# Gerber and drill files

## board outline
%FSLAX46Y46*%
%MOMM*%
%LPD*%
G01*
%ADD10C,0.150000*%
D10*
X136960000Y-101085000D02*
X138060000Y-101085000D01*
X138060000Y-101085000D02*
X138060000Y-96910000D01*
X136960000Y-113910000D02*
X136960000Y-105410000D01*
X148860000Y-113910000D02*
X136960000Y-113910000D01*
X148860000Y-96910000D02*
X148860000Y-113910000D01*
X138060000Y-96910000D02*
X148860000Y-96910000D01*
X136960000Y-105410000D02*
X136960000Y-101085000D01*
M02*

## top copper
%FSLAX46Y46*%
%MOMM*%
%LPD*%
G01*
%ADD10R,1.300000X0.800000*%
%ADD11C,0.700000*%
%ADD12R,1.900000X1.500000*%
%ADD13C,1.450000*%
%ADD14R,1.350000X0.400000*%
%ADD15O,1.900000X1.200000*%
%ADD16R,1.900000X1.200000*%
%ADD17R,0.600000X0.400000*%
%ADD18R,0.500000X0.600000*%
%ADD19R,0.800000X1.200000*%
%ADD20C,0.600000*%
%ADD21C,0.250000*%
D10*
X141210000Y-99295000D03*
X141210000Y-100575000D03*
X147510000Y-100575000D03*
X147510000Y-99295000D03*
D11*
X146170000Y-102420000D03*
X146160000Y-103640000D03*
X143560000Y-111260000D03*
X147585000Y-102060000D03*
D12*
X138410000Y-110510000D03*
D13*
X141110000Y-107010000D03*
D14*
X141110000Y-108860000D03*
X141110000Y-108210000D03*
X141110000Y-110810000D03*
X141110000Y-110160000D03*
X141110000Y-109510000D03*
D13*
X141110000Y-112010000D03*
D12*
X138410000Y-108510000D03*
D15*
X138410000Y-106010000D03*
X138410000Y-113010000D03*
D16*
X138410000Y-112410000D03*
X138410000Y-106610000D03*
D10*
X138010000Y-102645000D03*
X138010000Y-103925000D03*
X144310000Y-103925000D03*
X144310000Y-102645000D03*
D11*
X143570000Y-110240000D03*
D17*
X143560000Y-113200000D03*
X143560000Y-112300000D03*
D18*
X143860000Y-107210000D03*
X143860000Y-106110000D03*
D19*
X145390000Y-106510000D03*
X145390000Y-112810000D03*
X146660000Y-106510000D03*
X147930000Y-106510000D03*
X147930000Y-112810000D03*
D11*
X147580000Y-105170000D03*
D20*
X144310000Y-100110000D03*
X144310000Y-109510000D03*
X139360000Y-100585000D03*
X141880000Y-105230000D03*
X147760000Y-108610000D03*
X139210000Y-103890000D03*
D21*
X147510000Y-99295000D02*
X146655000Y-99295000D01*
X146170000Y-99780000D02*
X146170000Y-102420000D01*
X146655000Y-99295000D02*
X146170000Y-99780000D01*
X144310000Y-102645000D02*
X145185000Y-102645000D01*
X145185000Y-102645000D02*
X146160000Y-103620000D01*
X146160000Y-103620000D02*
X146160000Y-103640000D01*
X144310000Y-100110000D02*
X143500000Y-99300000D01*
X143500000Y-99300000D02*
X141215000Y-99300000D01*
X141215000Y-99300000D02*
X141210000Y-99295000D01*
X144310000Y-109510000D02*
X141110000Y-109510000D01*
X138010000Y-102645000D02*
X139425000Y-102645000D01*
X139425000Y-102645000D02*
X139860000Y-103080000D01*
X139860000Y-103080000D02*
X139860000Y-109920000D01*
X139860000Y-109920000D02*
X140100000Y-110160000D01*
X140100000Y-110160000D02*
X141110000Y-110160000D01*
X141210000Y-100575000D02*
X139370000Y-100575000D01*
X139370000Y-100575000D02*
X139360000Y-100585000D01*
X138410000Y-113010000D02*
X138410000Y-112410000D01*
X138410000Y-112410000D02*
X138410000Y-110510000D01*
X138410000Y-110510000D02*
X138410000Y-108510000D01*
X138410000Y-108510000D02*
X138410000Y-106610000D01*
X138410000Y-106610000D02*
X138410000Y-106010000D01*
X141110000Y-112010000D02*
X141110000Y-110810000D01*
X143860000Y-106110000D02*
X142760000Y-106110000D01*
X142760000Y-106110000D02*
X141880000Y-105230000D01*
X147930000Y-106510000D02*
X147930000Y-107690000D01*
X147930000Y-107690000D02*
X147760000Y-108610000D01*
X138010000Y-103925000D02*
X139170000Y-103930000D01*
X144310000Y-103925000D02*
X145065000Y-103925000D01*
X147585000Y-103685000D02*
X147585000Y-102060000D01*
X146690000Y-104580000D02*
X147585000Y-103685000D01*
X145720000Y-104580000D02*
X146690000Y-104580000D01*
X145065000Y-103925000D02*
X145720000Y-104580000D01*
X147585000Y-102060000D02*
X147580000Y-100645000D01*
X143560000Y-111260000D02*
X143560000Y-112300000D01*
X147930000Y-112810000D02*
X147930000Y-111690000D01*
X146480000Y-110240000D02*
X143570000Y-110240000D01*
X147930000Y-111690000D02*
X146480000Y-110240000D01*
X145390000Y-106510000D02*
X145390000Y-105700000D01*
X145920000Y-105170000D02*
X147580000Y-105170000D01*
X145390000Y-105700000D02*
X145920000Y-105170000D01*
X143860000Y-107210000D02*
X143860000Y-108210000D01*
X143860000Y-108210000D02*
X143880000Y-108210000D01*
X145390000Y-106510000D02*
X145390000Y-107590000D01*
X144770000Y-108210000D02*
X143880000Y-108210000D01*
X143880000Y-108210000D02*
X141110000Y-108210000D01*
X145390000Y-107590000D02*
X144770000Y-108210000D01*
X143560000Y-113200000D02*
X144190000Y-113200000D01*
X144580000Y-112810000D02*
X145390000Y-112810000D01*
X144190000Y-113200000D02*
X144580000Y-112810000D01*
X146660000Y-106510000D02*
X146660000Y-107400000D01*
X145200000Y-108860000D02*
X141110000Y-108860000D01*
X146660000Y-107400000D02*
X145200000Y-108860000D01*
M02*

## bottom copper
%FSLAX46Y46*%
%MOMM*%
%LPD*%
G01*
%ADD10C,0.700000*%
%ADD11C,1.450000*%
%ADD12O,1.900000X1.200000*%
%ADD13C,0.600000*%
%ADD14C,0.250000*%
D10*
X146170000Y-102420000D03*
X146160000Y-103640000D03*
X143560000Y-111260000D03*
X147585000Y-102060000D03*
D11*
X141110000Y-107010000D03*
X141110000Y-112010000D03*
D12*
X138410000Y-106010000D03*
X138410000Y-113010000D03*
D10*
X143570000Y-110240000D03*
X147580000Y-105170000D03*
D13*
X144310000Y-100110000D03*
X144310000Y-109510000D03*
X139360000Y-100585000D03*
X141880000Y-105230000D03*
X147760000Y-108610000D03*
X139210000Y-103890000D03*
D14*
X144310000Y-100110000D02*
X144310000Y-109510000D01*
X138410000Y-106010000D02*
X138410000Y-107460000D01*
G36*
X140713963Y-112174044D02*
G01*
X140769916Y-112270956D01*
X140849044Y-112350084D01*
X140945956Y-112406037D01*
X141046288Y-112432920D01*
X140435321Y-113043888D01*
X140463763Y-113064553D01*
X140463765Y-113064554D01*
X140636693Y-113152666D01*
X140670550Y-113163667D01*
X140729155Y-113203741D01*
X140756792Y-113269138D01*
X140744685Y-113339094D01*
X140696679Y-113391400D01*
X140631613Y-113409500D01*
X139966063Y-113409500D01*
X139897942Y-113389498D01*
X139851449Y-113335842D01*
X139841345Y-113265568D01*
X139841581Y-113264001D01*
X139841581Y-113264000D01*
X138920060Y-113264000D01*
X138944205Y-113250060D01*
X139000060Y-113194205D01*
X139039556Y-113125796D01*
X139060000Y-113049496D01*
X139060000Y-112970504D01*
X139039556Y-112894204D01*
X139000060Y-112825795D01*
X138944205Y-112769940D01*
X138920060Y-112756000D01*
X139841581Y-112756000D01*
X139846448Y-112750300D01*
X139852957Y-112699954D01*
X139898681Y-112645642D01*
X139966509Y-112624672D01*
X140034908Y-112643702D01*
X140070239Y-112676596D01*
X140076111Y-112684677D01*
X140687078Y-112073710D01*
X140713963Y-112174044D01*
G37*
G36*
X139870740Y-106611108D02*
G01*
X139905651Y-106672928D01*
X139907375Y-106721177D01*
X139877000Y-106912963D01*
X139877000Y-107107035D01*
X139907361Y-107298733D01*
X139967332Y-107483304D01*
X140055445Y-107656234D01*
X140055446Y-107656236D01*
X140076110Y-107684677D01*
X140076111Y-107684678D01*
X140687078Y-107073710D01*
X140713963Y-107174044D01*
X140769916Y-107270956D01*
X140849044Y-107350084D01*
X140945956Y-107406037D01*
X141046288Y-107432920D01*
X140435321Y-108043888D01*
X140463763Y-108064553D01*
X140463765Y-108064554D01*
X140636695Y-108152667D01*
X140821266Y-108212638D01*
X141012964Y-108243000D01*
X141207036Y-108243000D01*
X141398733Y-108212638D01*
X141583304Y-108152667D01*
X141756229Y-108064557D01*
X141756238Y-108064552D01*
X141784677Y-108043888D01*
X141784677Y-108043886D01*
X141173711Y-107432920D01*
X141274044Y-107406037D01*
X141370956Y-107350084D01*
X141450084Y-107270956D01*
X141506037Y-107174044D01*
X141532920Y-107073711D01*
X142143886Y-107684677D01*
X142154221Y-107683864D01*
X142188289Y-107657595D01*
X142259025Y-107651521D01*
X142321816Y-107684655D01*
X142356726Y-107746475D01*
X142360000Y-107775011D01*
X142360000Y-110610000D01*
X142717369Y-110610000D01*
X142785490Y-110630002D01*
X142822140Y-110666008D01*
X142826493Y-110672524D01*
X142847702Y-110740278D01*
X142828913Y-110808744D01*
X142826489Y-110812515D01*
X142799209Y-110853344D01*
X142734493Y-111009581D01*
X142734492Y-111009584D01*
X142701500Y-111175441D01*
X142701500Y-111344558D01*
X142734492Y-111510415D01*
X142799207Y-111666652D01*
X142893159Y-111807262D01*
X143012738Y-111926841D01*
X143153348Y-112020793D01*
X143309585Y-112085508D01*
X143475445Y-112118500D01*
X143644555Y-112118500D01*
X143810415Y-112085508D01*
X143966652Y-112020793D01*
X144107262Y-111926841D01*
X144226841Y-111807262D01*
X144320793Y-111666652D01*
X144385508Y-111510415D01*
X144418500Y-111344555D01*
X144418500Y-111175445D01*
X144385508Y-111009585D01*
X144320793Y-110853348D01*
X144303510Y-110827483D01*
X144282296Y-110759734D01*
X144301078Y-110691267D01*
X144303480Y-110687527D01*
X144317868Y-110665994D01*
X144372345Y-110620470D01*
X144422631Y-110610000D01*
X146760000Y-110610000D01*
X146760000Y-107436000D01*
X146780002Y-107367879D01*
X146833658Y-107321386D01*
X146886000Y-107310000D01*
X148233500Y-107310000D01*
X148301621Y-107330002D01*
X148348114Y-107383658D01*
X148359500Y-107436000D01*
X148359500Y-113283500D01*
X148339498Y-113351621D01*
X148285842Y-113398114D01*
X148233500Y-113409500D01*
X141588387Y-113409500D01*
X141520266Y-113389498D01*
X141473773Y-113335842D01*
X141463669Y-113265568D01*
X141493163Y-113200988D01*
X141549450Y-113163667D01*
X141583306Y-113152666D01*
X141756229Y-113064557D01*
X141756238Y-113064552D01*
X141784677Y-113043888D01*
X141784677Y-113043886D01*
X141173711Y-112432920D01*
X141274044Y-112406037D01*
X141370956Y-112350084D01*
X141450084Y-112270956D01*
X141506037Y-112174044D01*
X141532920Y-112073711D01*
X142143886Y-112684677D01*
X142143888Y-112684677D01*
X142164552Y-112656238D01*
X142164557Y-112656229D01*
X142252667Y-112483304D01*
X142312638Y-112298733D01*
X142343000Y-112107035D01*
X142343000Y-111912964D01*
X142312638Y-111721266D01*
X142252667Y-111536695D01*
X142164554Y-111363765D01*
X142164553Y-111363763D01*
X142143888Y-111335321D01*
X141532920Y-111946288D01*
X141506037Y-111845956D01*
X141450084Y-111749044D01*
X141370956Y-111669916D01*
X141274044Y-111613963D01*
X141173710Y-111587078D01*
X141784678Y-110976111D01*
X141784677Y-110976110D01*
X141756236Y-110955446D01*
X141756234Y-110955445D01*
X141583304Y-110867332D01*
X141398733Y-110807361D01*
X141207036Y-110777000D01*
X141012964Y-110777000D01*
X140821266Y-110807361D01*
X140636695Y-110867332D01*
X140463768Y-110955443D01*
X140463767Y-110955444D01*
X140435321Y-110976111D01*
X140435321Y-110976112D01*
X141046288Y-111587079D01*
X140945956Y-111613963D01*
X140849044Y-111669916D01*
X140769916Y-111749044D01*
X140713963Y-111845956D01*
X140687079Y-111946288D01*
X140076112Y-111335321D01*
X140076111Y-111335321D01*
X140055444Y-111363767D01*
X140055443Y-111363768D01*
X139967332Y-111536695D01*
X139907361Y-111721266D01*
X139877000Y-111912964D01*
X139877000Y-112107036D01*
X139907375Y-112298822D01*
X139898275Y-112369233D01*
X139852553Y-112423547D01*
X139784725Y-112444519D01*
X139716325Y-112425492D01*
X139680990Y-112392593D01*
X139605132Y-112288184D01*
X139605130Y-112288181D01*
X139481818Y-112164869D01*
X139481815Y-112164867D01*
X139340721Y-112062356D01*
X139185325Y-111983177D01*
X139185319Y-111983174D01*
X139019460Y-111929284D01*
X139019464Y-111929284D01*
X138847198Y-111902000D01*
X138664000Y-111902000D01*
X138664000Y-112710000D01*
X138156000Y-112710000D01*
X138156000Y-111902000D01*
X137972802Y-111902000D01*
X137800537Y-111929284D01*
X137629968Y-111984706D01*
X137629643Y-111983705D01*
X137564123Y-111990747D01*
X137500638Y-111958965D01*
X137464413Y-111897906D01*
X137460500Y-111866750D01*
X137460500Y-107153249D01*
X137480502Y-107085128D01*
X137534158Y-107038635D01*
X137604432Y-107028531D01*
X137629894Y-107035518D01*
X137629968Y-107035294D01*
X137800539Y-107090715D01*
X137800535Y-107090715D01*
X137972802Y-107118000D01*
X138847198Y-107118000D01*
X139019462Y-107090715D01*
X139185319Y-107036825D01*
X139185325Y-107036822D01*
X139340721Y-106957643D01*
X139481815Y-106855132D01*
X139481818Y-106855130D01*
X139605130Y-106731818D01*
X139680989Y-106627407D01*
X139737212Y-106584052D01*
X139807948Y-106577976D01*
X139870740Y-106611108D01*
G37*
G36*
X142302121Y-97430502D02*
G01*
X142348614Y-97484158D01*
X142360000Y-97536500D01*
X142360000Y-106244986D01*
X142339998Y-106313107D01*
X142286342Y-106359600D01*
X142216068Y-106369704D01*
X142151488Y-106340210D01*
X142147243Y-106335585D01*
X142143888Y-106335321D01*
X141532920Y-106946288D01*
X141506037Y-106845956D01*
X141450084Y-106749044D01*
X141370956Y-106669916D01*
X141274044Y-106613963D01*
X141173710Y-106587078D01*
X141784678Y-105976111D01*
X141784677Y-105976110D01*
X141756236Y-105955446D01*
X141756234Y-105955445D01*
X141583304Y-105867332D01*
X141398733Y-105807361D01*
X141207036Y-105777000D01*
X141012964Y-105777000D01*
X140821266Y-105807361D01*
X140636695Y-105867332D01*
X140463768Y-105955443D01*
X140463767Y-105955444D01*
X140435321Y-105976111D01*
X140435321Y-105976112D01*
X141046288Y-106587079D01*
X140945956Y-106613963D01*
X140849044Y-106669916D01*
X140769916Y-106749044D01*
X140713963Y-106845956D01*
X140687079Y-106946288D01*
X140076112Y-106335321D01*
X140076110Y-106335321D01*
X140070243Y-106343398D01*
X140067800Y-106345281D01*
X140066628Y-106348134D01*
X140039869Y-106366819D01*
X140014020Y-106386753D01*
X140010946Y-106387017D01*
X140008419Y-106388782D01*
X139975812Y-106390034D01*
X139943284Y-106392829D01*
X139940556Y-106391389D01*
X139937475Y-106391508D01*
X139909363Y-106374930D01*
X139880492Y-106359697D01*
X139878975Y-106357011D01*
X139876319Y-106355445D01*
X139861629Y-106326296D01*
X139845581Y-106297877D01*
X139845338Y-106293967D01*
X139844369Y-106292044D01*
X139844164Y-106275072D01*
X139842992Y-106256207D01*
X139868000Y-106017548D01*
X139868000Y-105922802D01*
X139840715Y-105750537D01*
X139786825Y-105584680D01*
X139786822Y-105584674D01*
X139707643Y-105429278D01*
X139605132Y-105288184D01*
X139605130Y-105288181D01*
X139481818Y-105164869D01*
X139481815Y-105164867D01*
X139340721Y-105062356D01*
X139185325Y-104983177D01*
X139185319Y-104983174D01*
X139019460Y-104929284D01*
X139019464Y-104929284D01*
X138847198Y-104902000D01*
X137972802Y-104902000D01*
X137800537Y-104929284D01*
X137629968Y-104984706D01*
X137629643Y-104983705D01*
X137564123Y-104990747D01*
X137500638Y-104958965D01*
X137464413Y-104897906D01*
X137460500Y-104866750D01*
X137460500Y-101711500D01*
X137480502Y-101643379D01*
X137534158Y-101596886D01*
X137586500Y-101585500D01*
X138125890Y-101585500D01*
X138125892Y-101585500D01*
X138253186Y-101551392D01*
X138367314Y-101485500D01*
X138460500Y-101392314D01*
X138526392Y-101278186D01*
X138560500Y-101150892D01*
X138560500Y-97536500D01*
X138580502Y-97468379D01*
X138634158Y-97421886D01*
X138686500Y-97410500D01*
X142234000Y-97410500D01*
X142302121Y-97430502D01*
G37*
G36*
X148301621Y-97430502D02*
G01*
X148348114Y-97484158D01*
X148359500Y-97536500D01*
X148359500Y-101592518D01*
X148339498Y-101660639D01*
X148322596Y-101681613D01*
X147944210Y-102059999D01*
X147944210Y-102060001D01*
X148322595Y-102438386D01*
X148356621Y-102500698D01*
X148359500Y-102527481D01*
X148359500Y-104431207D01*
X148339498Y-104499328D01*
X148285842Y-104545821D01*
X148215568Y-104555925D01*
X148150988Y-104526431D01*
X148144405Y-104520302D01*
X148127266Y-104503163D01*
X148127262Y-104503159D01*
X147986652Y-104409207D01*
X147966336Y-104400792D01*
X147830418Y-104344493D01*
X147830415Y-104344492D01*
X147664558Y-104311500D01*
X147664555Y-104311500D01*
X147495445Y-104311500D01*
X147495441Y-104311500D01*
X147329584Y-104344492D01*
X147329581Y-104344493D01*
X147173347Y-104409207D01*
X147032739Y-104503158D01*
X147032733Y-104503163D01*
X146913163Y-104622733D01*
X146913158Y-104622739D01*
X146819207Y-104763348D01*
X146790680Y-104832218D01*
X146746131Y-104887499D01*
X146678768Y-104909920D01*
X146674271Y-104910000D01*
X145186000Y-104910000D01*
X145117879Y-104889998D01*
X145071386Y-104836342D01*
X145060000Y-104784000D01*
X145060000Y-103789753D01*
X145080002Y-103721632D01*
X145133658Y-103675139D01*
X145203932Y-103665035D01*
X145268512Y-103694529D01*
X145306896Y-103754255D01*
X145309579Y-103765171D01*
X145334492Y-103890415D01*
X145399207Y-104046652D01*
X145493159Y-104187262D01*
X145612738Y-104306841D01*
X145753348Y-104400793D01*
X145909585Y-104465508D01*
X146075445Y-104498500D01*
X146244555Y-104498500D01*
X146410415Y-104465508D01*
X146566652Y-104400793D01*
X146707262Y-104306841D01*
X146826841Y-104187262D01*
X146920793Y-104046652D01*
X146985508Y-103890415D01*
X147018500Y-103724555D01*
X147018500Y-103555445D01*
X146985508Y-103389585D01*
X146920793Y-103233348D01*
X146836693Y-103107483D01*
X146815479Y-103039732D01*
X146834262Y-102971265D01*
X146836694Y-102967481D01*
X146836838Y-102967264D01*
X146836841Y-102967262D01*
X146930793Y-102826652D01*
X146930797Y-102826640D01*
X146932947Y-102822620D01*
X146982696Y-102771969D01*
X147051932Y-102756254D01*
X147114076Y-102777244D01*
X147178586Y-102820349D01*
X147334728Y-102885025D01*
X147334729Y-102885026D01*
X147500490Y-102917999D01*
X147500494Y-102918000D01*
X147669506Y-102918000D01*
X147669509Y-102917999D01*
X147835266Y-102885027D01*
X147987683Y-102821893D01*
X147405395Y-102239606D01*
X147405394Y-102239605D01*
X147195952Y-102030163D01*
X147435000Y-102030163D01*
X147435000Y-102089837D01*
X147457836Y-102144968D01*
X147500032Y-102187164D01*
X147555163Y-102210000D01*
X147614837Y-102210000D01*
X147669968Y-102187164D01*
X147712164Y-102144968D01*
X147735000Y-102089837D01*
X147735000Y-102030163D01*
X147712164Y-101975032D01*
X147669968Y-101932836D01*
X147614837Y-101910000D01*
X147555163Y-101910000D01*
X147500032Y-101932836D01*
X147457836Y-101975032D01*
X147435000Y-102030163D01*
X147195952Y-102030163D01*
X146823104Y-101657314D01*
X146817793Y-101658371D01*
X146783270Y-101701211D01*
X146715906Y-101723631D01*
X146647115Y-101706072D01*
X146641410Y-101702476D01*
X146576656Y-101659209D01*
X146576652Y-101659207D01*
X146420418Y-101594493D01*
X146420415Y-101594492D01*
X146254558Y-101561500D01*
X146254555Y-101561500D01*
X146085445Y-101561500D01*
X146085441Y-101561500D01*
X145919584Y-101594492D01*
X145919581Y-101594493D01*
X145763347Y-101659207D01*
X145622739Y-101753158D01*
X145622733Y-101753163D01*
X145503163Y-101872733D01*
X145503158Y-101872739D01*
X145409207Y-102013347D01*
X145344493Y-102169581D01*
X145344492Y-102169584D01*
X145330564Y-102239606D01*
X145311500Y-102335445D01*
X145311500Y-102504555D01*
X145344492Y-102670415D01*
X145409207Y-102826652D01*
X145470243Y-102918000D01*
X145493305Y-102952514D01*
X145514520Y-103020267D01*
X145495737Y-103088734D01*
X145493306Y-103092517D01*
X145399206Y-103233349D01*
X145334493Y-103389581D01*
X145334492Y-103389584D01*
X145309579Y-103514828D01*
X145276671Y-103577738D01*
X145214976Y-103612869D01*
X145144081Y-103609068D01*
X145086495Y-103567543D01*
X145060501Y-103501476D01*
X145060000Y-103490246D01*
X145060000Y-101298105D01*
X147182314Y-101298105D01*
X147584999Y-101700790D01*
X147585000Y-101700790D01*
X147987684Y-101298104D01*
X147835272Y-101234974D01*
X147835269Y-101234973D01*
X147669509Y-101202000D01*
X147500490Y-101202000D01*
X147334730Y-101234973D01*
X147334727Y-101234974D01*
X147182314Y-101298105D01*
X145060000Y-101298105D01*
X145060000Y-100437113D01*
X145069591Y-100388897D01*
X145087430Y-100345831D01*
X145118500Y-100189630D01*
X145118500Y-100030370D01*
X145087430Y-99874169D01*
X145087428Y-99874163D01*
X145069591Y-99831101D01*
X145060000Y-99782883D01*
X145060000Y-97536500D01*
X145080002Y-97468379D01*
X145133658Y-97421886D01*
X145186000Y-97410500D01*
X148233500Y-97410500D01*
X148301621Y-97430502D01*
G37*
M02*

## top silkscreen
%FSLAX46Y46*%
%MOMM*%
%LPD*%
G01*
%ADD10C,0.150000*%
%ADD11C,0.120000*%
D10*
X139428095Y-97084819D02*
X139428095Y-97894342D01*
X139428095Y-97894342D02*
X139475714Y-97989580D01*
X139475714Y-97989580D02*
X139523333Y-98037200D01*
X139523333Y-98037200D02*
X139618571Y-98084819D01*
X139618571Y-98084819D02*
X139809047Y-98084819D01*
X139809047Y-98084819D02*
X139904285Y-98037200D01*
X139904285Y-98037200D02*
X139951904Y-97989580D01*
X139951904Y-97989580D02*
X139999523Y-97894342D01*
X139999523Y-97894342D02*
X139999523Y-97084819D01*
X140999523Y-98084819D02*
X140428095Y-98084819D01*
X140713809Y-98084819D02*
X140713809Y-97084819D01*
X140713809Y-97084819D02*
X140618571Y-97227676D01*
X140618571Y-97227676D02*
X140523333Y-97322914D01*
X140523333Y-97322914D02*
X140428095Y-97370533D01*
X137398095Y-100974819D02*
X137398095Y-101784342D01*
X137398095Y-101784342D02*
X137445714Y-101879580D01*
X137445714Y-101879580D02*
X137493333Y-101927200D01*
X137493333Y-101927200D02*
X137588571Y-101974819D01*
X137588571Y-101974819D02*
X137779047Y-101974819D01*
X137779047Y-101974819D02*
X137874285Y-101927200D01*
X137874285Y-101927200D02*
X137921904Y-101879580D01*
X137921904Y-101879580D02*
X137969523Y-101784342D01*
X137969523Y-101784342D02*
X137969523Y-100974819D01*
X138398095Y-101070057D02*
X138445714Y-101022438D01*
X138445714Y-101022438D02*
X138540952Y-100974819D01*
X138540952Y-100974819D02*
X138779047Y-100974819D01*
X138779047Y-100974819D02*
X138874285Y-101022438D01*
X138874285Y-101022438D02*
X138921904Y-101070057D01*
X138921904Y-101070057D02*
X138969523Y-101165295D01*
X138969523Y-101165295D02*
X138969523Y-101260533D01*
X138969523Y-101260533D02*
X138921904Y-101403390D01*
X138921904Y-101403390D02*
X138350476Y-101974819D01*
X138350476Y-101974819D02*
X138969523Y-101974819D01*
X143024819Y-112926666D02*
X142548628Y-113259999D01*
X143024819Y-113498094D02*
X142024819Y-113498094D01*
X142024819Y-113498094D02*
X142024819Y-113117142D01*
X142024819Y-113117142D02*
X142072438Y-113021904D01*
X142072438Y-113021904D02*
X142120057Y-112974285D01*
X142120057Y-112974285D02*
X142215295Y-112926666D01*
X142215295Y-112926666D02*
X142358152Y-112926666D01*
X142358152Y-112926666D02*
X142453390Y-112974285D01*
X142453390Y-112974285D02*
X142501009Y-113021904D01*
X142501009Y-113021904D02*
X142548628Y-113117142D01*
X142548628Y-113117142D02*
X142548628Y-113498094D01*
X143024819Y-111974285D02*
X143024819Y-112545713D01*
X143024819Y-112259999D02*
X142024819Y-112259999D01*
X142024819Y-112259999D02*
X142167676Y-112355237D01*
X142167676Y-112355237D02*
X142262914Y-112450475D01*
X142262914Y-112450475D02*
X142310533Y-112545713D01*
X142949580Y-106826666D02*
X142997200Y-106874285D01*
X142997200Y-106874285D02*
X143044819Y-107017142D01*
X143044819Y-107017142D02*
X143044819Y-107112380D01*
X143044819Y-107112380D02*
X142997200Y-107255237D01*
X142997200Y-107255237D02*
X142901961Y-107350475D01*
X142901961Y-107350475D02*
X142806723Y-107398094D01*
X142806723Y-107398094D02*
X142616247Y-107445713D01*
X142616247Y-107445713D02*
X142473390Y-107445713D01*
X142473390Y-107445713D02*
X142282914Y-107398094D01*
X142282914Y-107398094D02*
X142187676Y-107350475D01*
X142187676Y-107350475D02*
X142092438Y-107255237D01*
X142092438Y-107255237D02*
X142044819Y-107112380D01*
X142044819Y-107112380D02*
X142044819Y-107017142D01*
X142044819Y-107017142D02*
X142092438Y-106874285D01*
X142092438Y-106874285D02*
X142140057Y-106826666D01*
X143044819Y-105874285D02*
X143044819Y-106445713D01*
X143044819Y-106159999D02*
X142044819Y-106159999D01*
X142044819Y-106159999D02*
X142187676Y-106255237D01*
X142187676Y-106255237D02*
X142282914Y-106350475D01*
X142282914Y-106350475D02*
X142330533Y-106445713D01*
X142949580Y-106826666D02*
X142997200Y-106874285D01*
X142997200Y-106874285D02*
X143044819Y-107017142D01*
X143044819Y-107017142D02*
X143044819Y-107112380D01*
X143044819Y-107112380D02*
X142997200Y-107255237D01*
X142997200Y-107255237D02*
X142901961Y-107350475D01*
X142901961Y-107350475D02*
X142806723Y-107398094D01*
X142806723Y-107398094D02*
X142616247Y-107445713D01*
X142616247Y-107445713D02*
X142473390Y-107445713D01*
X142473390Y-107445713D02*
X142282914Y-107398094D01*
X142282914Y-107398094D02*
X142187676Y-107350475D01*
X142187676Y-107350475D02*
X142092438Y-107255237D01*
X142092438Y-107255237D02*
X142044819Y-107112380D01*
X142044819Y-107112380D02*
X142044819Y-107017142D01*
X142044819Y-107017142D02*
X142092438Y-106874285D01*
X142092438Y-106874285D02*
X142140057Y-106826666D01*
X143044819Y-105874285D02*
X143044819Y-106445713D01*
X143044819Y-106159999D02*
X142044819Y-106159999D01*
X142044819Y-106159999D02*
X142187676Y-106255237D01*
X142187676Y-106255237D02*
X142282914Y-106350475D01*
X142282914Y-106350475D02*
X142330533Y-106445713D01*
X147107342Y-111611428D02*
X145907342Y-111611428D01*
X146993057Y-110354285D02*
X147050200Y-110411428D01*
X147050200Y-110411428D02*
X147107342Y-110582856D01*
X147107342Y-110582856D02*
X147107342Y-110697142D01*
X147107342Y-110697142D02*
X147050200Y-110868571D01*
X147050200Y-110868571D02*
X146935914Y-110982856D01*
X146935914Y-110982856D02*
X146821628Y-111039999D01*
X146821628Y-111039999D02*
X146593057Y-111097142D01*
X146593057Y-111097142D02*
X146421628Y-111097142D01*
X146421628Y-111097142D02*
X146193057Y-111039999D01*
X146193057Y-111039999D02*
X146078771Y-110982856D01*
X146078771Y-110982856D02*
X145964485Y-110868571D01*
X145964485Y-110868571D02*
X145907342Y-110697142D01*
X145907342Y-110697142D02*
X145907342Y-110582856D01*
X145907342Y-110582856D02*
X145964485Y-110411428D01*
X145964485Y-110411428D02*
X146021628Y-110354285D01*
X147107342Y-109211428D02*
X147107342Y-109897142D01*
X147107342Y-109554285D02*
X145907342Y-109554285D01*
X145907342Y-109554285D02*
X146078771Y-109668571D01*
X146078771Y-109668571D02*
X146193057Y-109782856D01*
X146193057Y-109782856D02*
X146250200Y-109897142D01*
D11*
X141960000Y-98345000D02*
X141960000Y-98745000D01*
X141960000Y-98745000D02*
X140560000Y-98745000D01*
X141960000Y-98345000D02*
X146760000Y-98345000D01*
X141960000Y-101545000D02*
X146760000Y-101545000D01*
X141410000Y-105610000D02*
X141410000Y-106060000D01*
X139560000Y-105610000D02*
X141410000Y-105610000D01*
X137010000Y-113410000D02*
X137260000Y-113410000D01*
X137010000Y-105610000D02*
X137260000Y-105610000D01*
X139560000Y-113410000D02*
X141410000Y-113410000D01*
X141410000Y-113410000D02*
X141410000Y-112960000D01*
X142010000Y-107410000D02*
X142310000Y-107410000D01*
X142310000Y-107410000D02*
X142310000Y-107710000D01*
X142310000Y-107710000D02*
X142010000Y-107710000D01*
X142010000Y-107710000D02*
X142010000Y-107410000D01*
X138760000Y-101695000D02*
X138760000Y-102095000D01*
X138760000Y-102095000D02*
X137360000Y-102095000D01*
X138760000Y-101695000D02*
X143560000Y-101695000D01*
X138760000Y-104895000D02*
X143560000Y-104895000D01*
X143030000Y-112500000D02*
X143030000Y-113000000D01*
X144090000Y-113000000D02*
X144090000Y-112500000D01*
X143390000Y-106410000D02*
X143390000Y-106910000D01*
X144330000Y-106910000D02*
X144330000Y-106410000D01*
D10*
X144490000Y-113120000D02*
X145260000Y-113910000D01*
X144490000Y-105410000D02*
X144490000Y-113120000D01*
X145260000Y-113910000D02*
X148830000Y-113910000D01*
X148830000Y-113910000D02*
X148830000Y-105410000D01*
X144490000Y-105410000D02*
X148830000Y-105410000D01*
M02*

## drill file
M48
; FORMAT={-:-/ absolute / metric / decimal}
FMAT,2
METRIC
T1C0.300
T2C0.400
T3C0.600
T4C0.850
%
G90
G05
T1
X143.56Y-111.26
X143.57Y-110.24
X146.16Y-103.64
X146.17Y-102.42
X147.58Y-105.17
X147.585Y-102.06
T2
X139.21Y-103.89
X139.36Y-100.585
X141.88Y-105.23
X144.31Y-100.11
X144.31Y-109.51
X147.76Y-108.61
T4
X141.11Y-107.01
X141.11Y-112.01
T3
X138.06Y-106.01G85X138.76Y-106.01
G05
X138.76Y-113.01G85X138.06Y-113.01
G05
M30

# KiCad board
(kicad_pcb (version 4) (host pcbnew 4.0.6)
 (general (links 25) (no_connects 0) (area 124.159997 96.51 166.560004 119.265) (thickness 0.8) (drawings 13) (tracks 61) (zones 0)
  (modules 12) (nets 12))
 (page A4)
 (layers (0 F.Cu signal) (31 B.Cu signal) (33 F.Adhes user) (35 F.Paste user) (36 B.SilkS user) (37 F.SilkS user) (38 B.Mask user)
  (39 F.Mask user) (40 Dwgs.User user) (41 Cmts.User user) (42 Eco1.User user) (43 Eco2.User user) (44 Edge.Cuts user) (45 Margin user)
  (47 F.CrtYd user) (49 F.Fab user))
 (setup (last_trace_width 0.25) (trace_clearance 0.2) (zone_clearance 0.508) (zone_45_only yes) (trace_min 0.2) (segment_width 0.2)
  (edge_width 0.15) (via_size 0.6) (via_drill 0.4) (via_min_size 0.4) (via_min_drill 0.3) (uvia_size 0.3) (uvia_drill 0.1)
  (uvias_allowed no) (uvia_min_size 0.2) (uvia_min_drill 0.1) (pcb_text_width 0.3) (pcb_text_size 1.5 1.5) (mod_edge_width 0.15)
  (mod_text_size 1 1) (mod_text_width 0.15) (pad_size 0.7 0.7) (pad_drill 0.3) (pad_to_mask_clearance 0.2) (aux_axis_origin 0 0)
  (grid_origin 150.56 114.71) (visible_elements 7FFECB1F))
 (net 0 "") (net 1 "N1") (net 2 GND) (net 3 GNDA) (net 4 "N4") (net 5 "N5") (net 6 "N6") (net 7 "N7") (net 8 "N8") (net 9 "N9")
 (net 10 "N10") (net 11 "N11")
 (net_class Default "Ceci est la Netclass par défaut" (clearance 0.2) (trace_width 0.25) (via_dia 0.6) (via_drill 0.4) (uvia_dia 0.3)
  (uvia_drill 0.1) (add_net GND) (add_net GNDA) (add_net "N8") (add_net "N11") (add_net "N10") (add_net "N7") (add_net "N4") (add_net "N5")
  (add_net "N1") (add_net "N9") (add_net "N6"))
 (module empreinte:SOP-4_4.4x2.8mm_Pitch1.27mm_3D (layer F.Cu) (at 144.36 99.935)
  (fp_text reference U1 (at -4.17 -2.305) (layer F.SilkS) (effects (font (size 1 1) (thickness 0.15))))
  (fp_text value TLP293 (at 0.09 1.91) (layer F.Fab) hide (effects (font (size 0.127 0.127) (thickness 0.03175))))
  (fp_line (start -2.4 -1.59) (end -2.4 -1.19) (layer F.SilkS) (width 0.12))
  (fp_line (start -2.4 -1.19) (end -3.8 -1.19) (layer F.SilkS) (width 0.12))
  (fp_line (start -2.4 -1.59) (end 2.4 -1.59) (layer F.SilkS) (width 0.12))
  (fp_line (start -2.4 1.61) (end 2.4 1.61) (layer F.SilkS) (width 0.12))
  (pad 1 smd rect (at -3.15 -0.64) (size 1.3 0.8) (layers F.Cu F.Paste F.Mask) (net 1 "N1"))
  (pad 2 smd rect (at -3.15 0.64) (size 1.3 0.8) (layers F.Cu F.Paste F.Mask) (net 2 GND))
  (pad 3 smd rect (at 3.15 0.64) (size 1.3 0.8) (layers F.Cu F.Paste F.Mask) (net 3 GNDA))
  (pad 4 smd rect (at 3.15 -0.64) (size 1.3 0.8) (layers F.Cu F.Paste F.Mask) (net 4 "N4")))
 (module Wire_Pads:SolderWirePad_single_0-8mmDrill (layer F.Cu) (at 146.17 102.42)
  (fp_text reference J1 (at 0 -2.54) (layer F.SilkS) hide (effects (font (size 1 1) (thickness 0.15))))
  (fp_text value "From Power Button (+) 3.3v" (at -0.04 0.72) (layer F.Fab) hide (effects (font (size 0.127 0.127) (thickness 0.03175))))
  (pad 1 thru_hole circle (at 0 0) (size 0.7 0.7) (drill 0.3) (layers *.Cu *.Mask) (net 4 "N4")))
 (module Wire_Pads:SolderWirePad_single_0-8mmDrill (layer F.Cu) (at 146.16 103.64)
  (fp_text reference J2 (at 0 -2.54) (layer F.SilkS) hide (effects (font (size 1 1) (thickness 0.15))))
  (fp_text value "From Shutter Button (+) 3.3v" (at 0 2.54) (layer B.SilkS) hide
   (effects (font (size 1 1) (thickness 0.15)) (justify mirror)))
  (pad 1 thru_hole circle (at 0 0) (size 0.7 0.7) (drill 0.3) (layers *.Cu *.Mask) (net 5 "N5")))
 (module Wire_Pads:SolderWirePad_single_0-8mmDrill (layer F.Cu) (at 143.56 111.26)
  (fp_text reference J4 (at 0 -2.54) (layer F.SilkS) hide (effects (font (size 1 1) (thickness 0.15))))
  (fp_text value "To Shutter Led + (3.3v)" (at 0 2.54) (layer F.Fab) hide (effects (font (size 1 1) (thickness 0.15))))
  (pad 1 thru_hole circle (at 0 0) (size 0.7 0.7) (drill 0.3) (layers *.Cu *.Mask) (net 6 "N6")))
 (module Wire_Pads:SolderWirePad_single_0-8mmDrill (layer F.Cu) (at 147.585 102.06)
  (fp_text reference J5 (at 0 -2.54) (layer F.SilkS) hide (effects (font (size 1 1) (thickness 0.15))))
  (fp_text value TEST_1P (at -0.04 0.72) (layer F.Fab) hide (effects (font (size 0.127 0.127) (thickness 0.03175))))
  (pad 1 thru_hole circle (at 0 0) (size 0.7 0.7) (drill 0.3) (layers *.Cu *.Mask) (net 3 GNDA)))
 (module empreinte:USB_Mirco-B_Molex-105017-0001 (layer F.Cu) (at 141.11 109.51 270)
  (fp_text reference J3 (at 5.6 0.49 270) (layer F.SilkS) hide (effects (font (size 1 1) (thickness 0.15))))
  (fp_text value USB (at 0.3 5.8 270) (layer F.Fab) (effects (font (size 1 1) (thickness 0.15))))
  (fp_line (start -3.9 -0.3) (end -3.45 -0.3) (layer F.SilkS) (width 0.12))
  (fp_line (start -3.9 1.55) (end -3.9 -0.3) (layer F.SilkS) (width 0.12))
  (fp_line (start 3.9 4.1) (end 3.9 3.85) (layer F.SilkS) (width 0.12))
  (fp_line (start -3.9 4.1) (end -3.9 3.85) (layer F.SilkS) (width 0.12))
  (fp_line (start 3.9 1.55) (end 3.9 -0.3) (layer F.SilkS) (width 0.12))
  (fp_line (start 3.9 -0.3) (end 3.45 -0.3) (layer F.SilkS) (width 0.12))
  (fp_line (start -2.1 -0.9) (end -2.1 -1.2) (layer F.SilkS) (width 0.12))
  (fp_line (start -2.1 -1.2) (end -1.8 -1.2) (layer F.SilkS) (width 0.12))
  (fp_line (start -1.8 -1.2) (end -1.8 -0.9) (layer F.SilkS) (width 0.12))
  (fp_line (start -1.8 -0.9) (end -2.1 -0.9) (layer F.SilkS) (width 0.12))
  (pad 6 smd rect (at 1 2.7 270) (size 1.5 1.9) (layers F.Cu F.Paste F.Mask) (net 2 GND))
  (pad 6 thru_hole circle (at -2.5 0 270) (size 1.45 1.45) (drill 0.85) (layers *.Cu *.Mask) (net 2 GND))
  (pad 2 smd rect (at -0.65 0 270) (size 0.4 1.35) (layers F.Cu F.Paste F.Mask) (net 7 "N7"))
  (pad 1 smd rect (at -1.3 0 270) (size 0.4 1.35) (layers F.Cu F.Paste F.Mask) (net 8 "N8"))
  (pad 5 smd rect (at 1.3 0 270) (size 0.4 1.35) (layers F.Cu F.Paste F.Mask) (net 2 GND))
  (pad 4 smd rect (at 0.65 0 270) (size 0.4 1.35) (layers F.Cu F.Paste F.Mask) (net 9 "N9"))
  (pad 3 smd rect (at 0 0 270) (size 0.4 1.35) (layers F.Cu F.Paste F.Mask) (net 1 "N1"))
  (pad 6 thru_hole circle (at 2.5 0 270) (size 1.45 1.45) (drill 0.85) (layers *.Cu *.Mask) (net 2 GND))
  (pad 6 smd rect (at -1 2.7 270) (size 1.5 1.9) (layers F.Cu F.Paste F.Mask) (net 2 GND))
  (pad 6 thru_hole oval (at -3.5 2.7 90) (size 1.2 1.9) (drill oval 0.6 1.3) (layers *.Cu *.Mask) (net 2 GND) (zone_connect 0))
  (pad 6 thru_hole oval (at 3.5 2.7 270) (size 1.2 1.9) (drill oval 0.6 1.3) (layers *.Cu *.Mask) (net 2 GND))
  (pad 6 smd rect (at 2.9 2.7 270) (size 1.2 1.9) (layers F.Cu F.Mask) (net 2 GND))
  (pad 6 smd rect (at -2.9 2.7 270) (size 1.2 1.9) (layers F.Cu F.Mask) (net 2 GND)))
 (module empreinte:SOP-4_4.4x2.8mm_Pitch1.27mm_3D (layer F.Cu) (at 141.16 103.285)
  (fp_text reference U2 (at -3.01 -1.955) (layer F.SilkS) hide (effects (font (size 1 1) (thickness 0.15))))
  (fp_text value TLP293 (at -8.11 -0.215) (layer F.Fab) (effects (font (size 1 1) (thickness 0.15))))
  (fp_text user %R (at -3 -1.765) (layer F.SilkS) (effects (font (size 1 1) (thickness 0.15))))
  (fp_line (start -2.4 -1.59) (end -2.4 -1.19) (layer F.SilkS) (width 0.12))
  (fp_line (start -2.4 -1.19) (end -3.8 -1.19) (layer F.SilkS) (width 0.12))
  (fp_line (start -2.4 -1.59) (end 2.4 -1.59) (layer F.SilkS) (width 0.12))
  (fp_line (start -2.4 1.61) (end 2.4 1.61) (layer F.SilkS) (width 0.12))
  (pad 1 smd rect (at -3.15 -0.64) (size 1.3 0.8) (layers F.Cu F.Paste F.Mask) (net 9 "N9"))
  (pad 2 smd rect (at -3.15 0.64) (size 1.3 0.8) (layers F.Cu F.Paste F.Mask) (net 2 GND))
  (pad 3 smd rect (at 3.15 0.64) (size 1.3 0.8) (layers F.Cu F.Paste F.Mask) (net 3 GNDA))
  (pad 4 smd rect (at 3.15 -0.64) (size 1.3 0.8) (layers F.Cu F.Paste F.Mask) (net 5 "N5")))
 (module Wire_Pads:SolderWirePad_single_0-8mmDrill (layer F.Cu) (at 143.57 110.24)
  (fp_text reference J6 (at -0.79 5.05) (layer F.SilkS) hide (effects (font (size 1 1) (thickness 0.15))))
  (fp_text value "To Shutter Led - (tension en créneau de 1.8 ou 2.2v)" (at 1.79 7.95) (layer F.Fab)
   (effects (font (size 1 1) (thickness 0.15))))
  (pad 1 thru_hole circle (at 0 0) (size 0.7 0.7) (drill 0.3) (layers *.Cu *.Mask) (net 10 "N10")))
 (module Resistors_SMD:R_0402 (layer F.Cu) (at 143.56 112.75 90)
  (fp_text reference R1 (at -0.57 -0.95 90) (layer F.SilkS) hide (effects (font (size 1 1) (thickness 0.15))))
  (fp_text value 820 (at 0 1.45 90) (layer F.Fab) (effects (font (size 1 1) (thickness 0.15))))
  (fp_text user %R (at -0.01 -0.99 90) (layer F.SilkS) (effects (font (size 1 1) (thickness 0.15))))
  (fp_line (start 0.25 -0.53) (end -0.25 -0.53) (layer F.SilkS) (width 0.12))
  (fp_line (start -0.25 0.53) (end 0.25 0.53) (layer F.SilkS) (width 0.12))
  (pad 1 smd rect (at -0.45 0 90) (size 0.4 0.6) (layers F.Cu F.Paste F.Mask) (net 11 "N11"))
  (pad 2 smd rect (at 0.45 0 90) (size 0.4 0.6) (layers F.Cu F.Paste F.Mask) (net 6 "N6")))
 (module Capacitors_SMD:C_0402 (layer F.Cu) (at 143.86 106.66 90)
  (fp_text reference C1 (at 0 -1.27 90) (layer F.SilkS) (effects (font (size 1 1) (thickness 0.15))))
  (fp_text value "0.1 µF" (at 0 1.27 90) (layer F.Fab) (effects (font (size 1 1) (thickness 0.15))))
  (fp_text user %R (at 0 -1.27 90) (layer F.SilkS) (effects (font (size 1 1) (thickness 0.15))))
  (fp_line (start 0.25 -0.47) (end -0.25 -0.47) (layer F.SilkS) (width 0.12))
  (fp_line (start -0.25 0.47) (end 0.25 0.47) (layer F.SilkS) (width 0.12))
  (pad 1 smd rect (at -0.55 0 90) (size 0.6 0.5) (layers F.Cu F.Paste F.Mask) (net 8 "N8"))
  (pad 2 smd rect (at 0.55 0 90) (size 0.6 0.5) (layers F.Cu F.Paste F.Mask) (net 2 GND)))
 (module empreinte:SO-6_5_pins (layer F.Cu) (at 146.66 109.66)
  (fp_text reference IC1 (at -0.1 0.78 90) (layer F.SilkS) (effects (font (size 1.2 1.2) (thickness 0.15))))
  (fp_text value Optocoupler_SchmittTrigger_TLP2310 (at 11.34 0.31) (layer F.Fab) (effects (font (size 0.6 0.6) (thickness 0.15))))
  (fp_line (start -2.17 3.46) (end -1.4 4.25) (layer F.SilkS) (width 0.15))
  (fp_line (start -2.17 -4.25) (end -2.17 3.46) (layer F.SilkS) (width 0.15))
  (fp_line (start -1.4 4.25) (end 2.17 4.25) (layer F.SilkS) (width 0.15))
  (fp_line (start 2.17 4.25) (end 2.17 -4.25) (layer F.SilkS) (width 0.15))
  (fp_line (start -2.17 -4.25) (end 2.17 -4.25) (layer F.SilkS) (width 0.15))
  (pad 6 smd rect (at -1.27 -3.15) (size 0.8 1.2) (layers F.Cu F.Paste F.Mask) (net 8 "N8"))
  (pad 1 smd rect (at -1.27 3.15) (size 0.8 1.2) (layers F.Cu F.Paste F.Mask) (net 11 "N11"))
  (pad 5 smd rect (at 0 -3.15) (size 0.8 1.2) (layers F.Cu F.Paste F.Mask) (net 7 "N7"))
  (pad 4 smd rect (at 1.27 -3.15) (size 0.8 1.2) (layers F.Cu F.Paste F.Mask) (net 2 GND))
  (pad 3 smd rect (at 1.27 3.15) (size 0.8 1.2) (layers F.Cu F.Paste F.Mask) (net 10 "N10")))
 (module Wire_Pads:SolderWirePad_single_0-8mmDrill (layer F.Cu) (at 147.58 105.17)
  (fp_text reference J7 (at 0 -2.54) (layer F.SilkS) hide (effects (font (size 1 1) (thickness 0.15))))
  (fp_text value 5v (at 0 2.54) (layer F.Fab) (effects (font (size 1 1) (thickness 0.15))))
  (pad 1 thru_hole circle (at 0 0) (size 0.7 0.7) (drill 0.3) (layers *.Cu *.Mask) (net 8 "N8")))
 (gr_line (start 136.96 101.085) (end 138.06 101.085) (layer Edge.Cuts) (width 0.15))
 (gr_line (start 138.06 101.085) (end 138.06 96.91) (angle 90) (layer Edge.Cuts) (width 0.15))
 (gr_line (start 136.96 113.91) (end 136.96 105.41) (angle 90) (layer Edge.Cuts) (width 0.15))
 (gr_line (start 148.86 113.91) (end 136.96 113.91) (angle 90) (layer Edge.Cuts) (width 0.15))
 (gr_line (start 148.86 96.91) (end 148.86 113.91) (angle 90) (layer Edge.Cuts) (width 0.15))
 (gr_line (start 138.06 96.91) (end 148.86 96.91) (angle 90) (layer Edge.Cuts) (width 0.15))
 (gr_line (start 136.96 105.41) (end 136.96 101.085) (angle 90) (layer Edge.Cuts) (width 0.15))
 (segment (start 147.51 99.295) (end 146.655 99.295) (width 0.25) (layer F.Cu) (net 4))
 (segment (start 146.17 99.78) (end 146.17 102.42) (width 0.25) (layer F.Cu) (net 4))
 (segment (start 146.655 99.295) (end 146.17 99.78) (width 0.25) (layer F.Cu) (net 4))
 (segment (start 144.31 102.645) (end 145.185 102.645) (width 0.25) (layer F.Cu) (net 5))
 (segment (start 145.185 102.645) (end 146.16 103.62) (width 0.25) (layer F.Cu) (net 5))
 (segment (start 146.16 103.62) (end 146.16 103.64) (width 0.25) (layer F.Cu) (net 5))
 (segment (start 144.31 100.11) (end 143.5 99.3) (width 0.25) (layer F.Cu) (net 1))
 (segment (start 143.5 99.3) (end 141.215 99.3) (width 0.25) (layer F.Cu) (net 1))
 (segment (start 141.215 99.3) (end 141.21 99.295) (width 0.25) (layer F.Cu) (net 1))
 (via (at 144.31 100.11) (size 0.6) (drill 0.4) (layers F.Cu B.Cu) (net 1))
 (segment (start 144.31 100.11) (end 144.31 109.51) (width 0.25) (layer B.Cu) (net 1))
 (via (at 144.31 109.51) (size 0.6) (drill 0.4) (layers F.Cu B.Cu) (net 1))
 (segment (start 144.31 109.51) (end 141.11 109.51) (width 0.25) (layer F.Cu) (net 1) (status 20))
 (segment (start 138.01 102.645) (end 139.425 102.645) (width 0.25) (layer F.Cu) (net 9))
 (segment (start 139.425 102.645) (end 139.86 103.08) (width 0.25) (layer F.Cu) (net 9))
 (segment (start 139.86 103.08) (end 139.86 109.92) (width 0.25) (layer F.Cu) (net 9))
 (segment (start 139.86 109.92) (end 140.1 110.16) (width 0.25) (layer F.Cu) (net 9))
 (segment (start 140.1 110.16) (end 141.11 110.16) (width 0.25) (layer F.Cu) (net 9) (status 20))
 (via (at 139.36 100.585) (size 0.6) (drill 0.4) (layers F.Cu B.Cu) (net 2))
 (segment (start 141.21 100.575) (end 139.37 100.575) (width 0.25) (layer F.Cu) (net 2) (status 10))
 (segment (start 139.37 100.575) (end 139.36 100.585) (width 0.25) (layer F.Cu) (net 2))
 (segment (start 138.41 113.01) (end 138.41 112.41) (width 0.25) (layer F.Cu) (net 2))
 (segment (start 138.41 112.41) (end 138.41 110.51) (width 0.25) (layer F.Cu) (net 2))
 (segment (start 138.41 110.51) (end 138.41 108.51) (width 0.25) (layer F.Cu) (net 2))
 (segment (start 138.41 108.51) (end 138.41 106.61) (width 0.25) (layer F.Cu) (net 2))
 (segment (start 138.41 106.61) (end 138.41 106.01) (width 0.25) (layer F.Cu) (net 2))
 (segment (start 138.41 106.01) (end 138.41 107.46) (width 0.25) (layer B.Cu) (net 2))
 (segment (start 141.11 112.01) (end 141.11 110.81) (width 0.25) (layer F.Cu) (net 2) (status 30))
 (segment (start 143.86 106.11) (end 142.76 106.11) (width 0.25) (layer F.Cu) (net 2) (status 10))
 (via (at 141.88 105.23) (size 0.6) (drill 0.4) (layers F.Cu B.Cu) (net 2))
 (segment (start 142.76 106.11) (end 141.88 105.23) (width 0.25) (layer F.Cu) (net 2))
 (segment (start 147.93 106.51) (end 147.93 107.69) (width 0.25) (layer F.Cu) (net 2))
 (via (at 147.76 108.61) (size 0.6) (drill 0.4) (layers F.Cu B.Cu) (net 2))
 (segment (start 147.93 107.69) (end 147.76 108.61) (width 0.25) (layer F.Cu) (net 2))
 (segment (start 138.01 103.925) (end 139.17 103.93) (width 0.25) (layer F.Cu) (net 2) (status 10))
 (via (at 139.21 103.89) (size 0.6) (drill 0.4) (layers F.Cu B.Cu) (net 2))
 (segment (start 144.31 103.925) (end 145.065 103.925) (width 0.25) (layer F.Cu) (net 3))
 (segment (start 147.585 103.685) (end 147.585 102.06) (width 0.25) (layer F.Cu) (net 3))
 (segment (start 146.69 104.58) (end 147.585 103.685) (width 0.25) (layer F.Cu) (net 3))
 (segment (start 145.72 104.58) (end 146.69 104.58) (width 0.25) (layer F.Cu) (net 3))
 (segment (start 145.065 103.925) (end 145.72 104.58) (width 0.25) (layer F.Cu) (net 3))
 (segment (start 147.585 102.06) (end 147.58 100.645) (width 0.25) (layer F.Cu) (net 3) (status 10))
 (segment (start 143.56 111.26) (end 143.56 112.3) (width 0.25) (layer F.Cu) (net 6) (status 10))
 (segment (start 147.93 112.81) (end 147.93 111.69) (width 0.25) (layer F.Cu) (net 10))
 (segment (start 146.48 110.24) (end 143.57 110.24) (width 0.25) (layer F.Cu) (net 10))
 (segment (start 147.93 111.69) (end 146.48 110.24) (width 0.25) (layer F.Cu) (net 10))
 (segment (start 145.39 106.51) (end 145.39 105.7) (width 0.25) (layer F.Cu) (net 8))
 (segment (start 145.92 105.17) (end 147.58 105.17) (width 0.25) (layer F.Cu) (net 8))
 (segment (start 145.39 105.7) (end 145.92 105.17) (width 0.25) (layer F.Cu) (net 8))
 (segment (start 143.86 107.21) (end 143.86 108.21) (width 0.25) (layer F.Cu) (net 8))
 (segment (start 143.86 108.21) (end 143.88 108.21) (width 0.25) (layer F.Cu) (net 8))
 (segment (start 145.39 106.51) (end 145.39 107.59) (width 0.25) (layer F.Cu) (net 8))
 (segment (start 144.77 108.21) (end 143.88 108.21) (width 0.25) (layer F.Cu) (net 8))
 (segment (start 143.88 108.21) (end 141.11 108.21) (width 0.25) (layer F.Cu) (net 8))
 (segment (start 145.39 107.59) (end 144.77 108.21) (width 0.25) (layer F.Cu) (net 8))
 (segment (start 143.56 113.2) (end 144.19 113.2) (width 0.25) (layer F.Cu) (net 11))
 (segment (start 144.58 112.81) (end 145.39 112.81) (width 0.25) (layer F.Cu) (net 11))
 (segment (start 144.19 113.2) (end 144.58 112.81) (width 0.25) (layer F.Cu) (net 11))
 (segment (start 146.66 106.51) (end 146.66 107.4) (width 0.25) (layer F.Cu) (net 7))
 (segment (start 145.2 108.86) (end 141.11 108.86) (width 0.25) (layer F.Cu) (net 7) (status 20))
 (segment (start 146.66 107.4) (end 145.2 108.86) (width 0.25) (layer F.Cu) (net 7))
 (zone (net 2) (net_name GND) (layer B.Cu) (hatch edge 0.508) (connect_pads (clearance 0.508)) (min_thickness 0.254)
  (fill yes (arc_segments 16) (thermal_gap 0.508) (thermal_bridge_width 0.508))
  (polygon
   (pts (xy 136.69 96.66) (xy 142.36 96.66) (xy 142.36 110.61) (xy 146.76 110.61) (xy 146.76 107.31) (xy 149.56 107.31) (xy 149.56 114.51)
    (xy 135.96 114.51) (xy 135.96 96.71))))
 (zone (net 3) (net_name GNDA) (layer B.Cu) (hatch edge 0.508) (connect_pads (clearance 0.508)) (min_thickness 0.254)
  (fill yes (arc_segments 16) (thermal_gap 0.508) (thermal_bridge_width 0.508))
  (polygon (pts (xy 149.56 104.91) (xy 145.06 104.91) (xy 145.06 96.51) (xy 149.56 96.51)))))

